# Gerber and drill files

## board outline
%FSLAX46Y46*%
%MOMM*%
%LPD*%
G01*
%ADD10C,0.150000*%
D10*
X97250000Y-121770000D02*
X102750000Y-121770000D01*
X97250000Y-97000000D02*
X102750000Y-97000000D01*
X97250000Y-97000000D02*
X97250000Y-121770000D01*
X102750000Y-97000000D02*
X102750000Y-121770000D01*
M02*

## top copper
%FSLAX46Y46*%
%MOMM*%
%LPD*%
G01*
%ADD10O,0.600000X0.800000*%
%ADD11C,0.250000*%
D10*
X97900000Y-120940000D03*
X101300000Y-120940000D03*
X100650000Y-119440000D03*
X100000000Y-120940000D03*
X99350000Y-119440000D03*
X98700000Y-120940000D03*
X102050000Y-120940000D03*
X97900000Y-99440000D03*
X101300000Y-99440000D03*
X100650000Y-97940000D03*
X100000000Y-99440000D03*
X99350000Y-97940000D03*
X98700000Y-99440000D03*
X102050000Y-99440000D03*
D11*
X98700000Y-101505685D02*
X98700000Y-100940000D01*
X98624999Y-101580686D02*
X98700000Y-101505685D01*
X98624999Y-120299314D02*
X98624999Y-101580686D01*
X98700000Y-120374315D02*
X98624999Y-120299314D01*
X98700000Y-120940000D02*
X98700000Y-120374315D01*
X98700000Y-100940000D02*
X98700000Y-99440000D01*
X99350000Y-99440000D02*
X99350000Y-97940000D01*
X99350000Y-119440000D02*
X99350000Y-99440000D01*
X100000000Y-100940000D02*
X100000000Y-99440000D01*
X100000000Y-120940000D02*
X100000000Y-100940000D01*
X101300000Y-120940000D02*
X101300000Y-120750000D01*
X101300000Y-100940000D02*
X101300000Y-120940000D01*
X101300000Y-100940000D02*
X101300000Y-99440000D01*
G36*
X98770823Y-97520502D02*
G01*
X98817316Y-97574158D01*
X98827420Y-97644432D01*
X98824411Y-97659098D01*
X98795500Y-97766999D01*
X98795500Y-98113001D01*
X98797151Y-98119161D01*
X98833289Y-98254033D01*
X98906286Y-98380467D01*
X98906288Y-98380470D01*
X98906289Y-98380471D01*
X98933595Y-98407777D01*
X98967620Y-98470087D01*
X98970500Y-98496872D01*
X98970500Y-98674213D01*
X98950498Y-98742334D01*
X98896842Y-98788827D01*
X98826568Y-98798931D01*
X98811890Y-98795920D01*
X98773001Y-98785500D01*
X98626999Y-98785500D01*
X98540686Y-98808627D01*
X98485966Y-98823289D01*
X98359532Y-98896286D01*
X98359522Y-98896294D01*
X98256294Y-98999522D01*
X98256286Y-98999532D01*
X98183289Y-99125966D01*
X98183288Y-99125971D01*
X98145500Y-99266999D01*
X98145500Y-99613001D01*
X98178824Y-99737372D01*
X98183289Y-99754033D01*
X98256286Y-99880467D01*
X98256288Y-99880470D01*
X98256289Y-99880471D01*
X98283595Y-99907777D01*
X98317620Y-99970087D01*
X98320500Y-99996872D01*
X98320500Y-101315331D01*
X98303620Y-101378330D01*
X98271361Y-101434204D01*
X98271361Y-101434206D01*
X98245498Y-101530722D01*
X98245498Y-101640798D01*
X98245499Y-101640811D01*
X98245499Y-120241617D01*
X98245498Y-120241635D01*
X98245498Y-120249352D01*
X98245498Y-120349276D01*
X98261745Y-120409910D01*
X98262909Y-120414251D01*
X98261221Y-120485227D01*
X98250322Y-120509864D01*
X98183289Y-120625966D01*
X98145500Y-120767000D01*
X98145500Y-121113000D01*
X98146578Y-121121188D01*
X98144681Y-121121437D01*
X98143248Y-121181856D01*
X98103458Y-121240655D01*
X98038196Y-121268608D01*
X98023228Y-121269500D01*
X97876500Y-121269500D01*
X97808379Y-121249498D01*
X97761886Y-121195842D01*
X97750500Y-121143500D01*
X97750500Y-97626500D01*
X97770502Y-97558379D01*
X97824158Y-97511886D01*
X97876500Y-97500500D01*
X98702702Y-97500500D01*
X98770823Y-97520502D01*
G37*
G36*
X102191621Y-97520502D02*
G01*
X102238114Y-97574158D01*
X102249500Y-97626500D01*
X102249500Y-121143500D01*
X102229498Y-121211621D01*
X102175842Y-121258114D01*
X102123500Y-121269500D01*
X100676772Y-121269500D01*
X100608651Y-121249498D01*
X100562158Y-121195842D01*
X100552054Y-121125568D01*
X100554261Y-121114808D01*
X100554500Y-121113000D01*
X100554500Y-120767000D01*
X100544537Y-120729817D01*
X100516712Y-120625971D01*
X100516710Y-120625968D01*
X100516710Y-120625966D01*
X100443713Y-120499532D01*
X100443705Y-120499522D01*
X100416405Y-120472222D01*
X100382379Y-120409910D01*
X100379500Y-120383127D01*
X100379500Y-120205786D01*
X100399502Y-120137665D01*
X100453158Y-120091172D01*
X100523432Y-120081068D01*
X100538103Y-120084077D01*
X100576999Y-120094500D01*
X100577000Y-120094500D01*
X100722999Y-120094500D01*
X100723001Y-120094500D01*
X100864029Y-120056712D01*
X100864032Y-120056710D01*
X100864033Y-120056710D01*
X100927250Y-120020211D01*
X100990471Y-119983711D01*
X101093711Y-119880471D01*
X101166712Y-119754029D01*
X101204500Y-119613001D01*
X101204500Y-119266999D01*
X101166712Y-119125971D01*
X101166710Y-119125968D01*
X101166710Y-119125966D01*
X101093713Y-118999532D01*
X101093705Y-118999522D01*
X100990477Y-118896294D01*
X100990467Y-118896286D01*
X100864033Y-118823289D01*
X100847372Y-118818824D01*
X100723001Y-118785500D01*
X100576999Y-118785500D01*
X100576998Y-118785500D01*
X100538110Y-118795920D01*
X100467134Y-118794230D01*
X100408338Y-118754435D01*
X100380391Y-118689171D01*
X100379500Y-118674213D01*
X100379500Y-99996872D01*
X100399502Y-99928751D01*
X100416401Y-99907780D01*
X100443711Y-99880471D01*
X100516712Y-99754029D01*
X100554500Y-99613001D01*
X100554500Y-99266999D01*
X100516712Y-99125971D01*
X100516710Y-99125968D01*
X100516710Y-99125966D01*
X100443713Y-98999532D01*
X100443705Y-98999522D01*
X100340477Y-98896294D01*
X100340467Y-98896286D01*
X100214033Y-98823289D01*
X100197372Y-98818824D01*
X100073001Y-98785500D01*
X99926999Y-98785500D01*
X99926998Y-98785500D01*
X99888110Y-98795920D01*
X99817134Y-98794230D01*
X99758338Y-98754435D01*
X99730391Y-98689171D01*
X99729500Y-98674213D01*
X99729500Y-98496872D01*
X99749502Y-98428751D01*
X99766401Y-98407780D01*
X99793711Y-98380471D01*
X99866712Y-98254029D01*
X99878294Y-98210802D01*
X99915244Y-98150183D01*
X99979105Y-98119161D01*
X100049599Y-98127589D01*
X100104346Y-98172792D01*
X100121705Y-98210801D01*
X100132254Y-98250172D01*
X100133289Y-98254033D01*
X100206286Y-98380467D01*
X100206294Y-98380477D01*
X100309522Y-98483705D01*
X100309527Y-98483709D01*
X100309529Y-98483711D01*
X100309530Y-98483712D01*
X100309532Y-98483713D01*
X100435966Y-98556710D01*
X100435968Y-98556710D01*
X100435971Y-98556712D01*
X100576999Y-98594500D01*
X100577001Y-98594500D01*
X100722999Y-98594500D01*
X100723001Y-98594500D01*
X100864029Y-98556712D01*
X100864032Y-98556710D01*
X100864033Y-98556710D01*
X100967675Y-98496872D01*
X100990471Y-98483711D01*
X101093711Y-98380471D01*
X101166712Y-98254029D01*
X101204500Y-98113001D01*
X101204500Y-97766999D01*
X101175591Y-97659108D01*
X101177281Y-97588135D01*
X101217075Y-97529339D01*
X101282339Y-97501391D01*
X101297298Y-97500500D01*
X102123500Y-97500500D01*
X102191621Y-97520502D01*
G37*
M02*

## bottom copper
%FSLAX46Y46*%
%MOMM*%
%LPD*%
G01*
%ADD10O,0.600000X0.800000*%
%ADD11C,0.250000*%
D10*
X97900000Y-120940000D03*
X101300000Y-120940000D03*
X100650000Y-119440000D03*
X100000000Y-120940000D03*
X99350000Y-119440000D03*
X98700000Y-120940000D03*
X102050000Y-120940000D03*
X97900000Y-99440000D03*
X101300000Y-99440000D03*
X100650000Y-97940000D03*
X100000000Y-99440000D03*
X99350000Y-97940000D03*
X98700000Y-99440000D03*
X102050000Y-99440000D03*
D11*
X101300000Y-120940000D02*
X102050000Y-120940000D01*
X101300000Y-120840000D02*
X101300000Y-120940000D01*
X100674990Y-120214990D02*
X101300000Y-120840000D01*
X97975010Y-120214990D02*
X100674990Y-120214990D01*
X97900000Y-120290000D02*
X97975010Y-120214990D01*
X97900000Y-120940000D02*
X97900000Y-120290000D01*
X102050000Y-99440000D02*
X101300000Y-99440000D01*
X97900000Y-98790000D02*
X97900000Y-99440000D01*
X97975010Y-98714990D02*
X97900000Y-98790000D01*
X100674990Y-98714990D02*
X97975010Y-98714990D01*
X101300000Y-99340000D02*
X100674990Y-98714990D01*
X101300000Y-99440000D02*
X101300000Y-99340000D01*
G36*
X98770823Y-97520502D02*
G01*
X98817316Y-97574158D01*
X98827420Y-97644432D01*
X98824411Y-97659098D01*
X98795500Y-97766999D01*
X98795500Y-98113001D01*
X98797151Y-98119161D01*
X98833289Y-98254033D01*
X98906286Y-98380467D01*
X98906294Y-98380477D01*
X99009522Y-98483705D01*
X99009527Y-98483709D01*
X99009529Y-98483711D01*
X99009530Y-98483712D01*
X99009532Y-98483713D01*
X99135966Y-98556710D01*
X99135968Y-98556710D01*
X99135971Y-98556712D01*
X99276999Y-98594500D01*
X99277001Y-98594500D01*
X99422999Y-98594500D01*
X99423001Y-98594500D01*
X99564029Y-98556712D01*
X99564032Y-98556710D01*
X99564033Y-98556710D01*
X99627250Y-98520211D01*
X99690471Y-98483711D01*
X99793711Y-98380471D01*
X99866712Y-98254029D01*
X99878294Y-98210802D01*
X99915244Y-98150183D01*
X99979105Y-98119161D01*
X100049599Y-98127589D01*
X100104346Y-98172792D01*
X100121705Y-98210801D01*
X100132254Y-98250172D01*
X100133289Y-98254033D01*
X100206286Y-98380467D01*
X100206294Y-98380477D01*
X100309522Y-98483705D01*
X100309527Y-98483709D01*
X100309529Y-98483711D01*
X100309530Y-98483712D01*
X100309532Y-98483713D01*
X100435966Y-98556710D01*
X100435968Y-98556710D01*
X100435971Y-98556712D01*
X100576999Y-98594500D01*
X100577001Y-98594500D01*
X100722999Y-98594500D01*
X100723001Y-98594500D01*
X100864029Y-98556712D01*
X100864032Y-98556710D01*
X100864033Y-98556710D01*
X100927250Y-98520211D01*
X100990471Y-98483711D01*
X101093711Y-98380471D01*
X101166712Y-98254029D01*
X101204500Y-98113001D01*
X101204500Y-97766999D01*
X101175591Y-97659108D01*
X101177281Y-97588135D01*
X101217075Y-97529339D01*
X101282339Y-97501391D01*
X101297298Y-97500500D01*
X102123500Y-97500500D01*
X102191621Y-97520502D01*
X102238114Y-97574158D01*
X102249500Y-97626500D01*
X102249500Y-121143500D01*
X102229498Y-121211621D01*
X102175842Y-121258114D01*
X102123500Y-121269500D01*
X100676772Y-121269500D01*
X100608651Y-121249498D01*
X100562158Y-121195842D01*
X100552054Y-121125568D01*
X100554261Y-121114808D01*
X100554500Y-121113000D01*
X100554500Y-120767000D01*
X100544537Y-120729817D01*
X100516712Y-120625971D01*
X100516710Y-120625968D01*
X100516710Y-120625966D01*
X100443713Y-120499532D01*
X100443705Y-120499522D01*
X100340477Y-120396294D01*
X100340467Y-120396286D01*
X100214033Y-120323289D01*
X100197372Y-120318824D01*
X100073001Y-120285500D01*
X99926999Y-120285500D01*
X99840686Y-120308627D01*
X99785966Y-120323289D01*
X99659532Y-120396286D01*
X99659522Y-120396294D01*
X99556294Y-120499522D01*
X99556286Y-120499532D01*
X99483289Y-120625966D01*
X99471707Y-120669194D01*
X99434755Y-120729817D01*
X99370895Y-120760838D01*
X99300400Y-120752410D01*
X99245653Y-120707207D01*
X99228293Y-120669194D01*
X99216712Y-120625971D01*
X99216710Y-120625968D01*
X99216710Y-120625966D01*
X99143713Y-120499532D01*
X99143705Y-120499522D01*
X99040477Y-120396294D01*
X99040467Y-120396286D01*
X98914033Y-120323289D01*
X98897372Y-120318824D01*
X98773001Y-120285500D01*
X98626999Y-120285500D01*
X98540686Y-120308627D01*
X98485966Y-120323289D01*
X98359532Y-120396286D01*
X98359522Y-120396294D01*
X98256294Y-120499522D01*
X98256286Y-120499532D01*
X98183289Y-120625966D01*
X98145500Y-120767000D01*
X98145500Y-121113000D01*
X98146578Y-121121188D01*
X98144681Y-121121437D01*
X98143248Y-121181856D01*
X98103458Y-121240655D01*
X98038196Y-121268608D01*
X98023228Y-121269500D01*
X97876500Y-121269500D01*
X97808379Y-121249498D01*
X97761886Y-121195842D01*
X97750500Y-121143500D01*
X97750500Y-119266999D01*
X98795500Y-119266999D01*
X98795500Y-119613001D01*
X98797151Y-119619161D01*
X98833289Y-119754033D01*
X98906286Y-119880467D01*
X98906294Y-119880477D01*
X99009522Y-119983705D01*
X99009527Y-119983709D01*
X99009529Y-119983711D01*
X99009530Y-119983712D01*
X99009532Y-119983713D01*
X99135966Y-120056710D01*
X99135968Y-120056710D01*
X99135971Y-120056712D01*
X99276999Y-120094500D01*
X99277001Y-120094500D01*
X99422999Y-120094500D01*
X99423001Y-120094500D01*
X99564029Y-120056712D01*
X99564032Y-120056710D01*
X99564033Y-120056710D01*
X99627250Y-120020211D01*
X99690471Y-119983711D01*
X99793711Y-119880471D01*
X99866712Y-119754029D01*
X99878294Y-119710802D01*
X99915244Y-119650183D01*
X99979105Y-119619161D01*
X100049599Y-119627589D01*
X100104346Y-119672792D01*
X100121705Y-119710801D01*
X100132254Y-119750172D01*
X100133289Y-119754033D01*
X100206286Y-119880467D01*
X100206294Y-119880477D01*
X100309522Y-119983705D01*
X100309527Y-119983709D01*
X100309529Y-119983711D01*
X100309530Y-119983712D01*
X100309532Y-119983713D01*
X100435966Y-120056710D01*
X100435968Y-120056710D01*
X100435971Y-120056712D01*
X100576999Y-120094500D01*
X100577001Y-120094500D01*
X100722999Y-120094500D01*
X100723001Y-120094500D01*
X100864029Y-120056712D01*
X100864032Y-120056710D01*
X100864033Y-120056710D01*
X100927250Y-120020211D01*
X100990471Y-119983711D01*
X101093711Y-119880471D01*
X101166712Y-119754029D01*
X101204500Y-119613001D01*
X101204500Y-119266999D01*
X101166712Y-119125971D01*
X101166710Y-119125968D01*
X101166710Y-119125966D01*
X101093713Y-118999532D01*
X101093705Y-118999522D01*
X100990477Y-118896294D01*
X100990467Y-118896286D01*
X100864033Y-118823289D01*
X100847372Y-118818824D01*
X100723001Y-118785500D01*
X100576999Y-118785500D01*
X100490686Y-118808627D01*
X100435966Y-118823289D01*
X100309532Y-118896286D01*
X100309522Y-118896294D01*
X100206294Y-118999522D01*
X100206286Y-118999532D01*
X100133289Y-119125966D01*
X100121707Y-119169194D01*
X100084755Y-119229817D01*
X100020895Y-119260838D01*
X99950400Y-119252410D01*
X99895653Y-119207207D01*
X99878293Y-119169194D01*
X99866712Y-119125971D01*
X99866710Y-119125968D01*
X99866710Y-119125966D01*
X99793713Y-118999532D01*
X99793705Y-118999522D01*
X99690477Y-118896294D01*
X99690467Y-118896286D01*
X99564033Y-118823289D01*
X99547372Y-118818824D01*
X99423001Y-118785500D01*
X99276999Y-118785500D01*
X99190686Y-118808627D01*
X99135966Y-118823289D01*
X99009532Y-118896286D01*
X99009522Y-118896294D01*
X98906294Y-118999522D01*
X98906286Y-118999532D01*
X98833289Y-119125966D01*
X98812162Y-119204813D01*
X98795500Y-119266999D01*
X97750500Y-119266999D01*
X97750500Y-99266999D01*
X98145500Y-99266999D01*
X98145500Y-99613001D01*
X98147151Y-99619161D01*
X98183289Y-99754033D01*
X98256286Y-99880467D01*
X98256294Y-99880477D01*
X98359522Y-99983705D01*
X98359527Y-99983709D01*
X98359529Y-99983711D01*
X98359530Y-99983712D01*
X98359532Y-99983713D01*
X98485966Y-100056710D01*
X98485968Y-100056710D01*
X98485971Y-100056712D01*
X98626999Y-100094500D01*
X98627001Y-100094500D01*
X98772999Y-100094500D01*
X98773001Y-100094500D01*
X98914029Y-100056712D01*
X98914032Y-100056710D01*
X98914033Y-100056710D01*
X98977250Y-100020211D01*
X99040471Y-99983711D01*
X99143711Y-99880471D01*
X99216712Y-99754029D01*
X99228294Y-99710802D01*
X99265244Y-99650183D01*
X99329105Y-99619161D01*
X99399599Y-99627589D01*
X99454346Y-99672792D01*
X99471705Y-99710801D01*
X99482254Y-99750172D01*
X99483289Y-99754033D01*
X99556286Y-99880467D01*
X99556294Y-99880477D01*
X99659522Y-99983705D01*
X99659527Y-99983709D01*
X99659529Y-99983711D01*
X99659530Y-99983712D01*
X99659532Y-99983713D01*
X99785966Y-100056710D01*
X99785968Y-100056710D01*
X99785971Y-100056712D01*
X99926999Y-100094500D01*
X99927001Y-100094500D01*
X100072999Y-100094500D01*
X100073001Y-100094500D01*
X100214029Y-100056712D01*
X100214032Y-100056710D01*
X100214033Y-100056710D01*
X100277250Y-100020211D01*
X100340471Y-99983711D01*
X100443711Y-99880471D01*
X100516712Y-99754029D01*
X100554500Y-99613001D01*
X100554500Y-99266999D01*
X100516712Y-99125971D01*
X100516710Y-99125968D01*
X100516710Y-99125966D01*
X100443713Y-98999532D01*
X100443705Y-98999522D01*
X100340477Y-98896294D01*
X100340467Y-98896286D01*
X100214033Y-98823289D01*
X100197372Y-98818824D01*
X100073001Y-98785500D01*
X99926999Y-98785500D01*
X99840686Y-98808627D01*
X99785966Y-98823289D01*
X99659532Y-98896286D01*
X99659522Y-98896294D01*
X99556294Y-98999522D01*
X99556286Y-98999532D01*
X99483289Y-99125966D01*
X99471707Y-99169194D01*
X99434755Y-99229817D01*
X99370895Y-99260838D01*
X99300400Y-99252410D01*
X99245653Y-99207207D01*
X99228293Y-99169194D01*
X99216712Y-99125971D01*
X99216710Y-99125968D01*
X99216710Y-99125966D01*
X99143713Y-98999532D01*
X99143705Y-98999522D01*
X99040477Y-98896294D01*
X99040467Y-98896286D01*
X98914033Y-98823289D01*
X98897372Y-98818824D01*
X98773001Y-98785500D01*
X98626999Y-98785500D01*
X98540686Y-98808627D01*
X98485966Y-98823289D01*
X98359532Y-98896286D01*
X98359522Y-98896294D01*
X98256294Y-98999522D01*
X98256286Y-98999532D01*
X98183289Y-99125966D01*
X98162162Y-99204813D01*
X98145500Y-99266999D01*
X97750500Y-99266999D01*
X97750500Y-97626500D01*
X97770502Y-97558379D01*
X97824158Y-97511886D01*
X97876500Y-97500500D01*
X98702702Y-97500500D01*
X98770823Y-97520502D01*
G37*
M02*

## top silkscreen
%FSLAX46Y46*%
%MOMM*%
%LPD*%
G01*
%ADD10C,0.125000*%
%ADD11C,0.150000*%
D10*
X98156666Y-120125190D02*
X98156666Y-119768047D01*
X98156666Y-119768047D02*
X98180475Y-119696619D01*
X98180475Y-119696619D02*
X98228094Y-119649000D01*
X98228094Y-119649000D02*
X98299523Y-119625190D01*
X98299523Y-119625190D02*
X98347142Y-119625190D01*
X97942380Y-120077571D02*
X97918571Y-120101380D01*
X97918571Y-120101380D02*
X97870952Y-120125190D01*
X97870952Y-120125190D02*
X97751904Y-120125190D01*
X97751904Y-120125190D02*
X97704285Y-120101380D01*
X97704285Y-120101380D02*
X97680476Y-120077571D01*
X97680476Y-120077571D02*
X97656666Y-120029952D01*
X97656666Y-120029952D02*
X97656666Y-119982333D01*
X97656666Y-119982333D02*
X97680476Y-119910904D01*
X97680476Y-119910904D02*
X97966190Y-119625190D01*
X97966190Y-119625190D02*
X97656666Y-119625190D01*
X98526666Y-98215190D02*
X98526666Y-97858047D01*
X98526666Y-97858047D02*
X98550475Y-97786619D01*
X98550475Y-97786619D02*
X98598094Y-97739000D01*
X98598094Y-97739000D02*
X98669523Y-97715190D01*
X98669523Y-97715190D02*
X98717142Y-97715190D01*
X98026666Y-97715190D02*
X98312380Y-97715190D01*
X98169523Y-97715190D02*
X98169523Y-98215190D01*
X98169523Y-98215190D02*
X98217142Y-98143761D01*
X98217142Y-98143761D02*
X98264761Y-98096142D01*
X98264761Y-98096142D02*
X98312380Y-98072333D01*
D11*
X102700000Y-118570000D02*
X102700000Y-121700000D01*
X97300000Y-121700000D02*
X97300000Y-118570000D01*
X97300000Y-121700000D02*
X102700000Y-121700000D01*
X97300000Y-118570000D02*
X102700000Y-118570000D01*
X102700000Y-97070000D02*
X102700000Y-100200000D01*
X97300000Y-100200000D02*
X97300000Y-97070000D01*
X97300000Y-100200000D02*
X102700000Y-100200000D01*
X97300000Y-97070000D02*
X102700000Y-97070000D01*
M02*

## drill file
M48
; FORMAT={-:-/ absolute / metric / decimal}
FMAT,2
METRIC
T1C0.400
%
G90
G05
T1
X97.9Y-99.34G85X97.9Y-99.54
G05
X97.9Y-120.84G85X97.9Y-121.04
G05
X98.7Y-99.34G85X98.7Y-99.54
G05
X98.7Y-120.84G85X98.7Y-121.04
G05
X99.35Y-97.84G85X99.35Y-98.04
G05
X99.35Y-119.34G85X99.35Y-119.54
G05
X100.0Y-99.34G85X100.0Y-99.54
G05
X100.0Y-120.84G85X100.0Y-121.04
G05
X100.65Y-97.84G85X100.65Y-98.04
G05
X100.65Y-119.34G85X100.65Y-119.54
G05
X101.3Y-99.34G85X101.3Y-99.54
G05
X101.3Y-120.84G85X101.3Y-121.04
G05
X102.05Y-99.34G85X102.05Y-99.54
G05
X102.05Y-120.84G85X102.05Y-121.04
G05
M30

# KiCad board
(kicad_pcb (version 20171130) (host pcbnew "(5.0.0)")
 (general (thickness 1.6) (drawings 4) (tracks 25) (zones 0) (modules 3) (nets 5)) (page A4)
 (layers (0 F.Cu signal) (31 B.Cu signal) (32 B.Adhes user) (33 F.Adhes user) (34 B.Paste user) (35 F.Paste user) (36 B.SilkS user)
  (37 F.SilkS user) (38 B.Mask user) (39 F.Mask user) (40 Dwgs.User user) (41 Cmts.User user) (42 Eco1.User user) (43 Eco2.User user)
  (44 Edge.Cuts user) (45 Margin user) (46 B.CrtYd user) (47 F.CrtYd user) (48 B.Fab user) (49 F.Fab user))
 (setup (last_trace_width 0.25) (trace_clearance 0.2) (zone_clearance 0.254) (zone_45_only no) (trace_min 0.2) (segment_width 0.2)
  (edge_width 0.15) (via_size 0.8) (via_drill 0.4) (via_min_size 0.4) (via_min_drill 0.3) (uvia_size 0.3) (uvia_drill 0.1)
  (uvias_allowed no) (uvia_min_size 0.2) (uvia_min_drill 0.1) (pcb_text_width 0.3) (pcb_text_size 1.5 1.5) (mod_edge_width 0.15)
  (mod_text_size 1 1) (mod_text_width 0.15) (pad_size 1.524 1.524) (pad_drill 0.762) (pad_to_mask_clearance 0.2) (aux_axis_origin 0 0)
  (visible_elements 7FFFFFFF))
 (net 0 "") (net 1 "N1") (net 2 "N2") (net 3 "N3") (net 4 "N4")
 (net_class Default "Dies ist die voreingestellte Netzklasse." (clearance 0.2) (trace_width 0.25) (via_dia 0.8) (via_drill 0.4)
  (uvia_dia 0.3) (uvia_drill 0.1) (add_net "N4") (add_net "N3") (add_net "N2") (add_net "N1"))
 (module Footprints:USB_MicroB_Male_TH (layer F.Cu) (at 100 120)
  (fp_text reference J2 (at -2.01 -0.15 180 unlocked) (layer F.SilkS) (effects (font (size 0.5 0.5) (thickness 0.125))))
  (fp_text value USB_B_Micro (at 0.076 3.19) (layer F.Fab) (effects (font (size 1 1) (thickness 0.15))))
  (fp_line (start 2.7 -1.43) (end 2.7 1.7) (layer F.SilkS) (width 0.15))
  (fp_line (start -2.7 1.7) (end -2.7 -1.43) (layer F.SilkS) (width 0.15))
  (fp_line (start -2.7 1.7) (end 2.7 1.7) (layer F.SilkS) (width 0.15))
  (fp_line (start -2.7 -1.43) (end 2.7 -1.43) (layer F.SilkS) (width 0.15))
  (pad 6 thru_hole oval (at -2.1 0.94) (size 0.6 0.8) (drill oval 0.4 0.6) (layers *.Cu *.Mask) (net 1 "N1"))
  (pad 5 thru_hole oval (at 1.3 0.94) (size 0.6 0.8) (drill oval 0.4 0.6) (layers *.Cu *.Mask) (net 1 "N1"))
  (pad 4 thru_hole oval (at 0.65 -0.56) (size 0.6 0.8) (drill oval 0.4 0.6) (layers *.Cu *.Mask))
  (pad 3 thru_hole oval (at 0 0.94) (size 0.6 0.8) (drill oval 0.4 0.6) (layers *.Cu *.Mask) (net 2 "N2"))
  (pad 2 thru_hole oval (at -0.65 -0.56) (size 0.6 0.8) (drill oval 0.4 0.6) (layers *.Cu *.Mask) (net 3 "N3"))
  (pad 1 thru_hole oval (at -1.3 0.94) (size 0.6 0.8) (drill oval 0.4 0.6) (layers *.Cu *.Mask) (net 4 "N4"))
  (pad 6 thru_hole oval (at 2.05 0.94) (size 0.6 0.8) (drill oval 0.4 0.6) (layers *.Cu *.Mask) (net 1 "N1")))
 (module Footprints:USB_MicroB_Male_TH (layer F.Cu) (at 100 98.5)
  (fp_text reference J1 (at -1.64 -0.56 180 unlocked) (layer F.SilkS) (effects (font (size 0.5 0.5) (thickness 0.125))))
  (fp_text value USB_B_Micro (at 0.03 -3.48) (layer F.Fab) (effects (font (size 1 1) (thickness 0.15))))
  (fp_line (start 2.7 -1.43) (end 2.7 1.7) (layer F.SilkS) (width 0.15))
  (fp_line (start -2.7 1.7) (end -2.7 -1.43) (layer F.SilkS) (width 0.15))
  (fp_line (start -2.7 1.7) (end 2.7 1.7) (layer F.SilkS) (width 0.15))
  (fp_line (start -2.7 -1.43) (end 2.7 -1.43) (layer F.SilkS) (width 0.15))
  (pad 6 thru_hole oval (at -2.1 0.94) (size 0.6 0.8) (drill oval 0.4 0.6) (layers *.Cu *.Mask) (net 1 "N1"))
  (pad 5 thru_hole oval (at 1.3 0.94) (size 0.6 0.8) (drill oval 0.4 0.6) (layers *.Cu *.Mask) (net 1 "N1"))
  (pad 4 thru_hole oval (at 0.65 -0.56) (size 0.6 0.8) (drill oval 0.4 0.6) (layers *.Cu *.Mask))
  (pad 3 thru_hole oval (at 0 0.94) (size 0.6 0.8) (drill oval 0.4 0.6) (layers *.Cu *.Mask) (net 2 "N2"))
  (pad 2 thru_hole oval (at -0.65 -0.56) (size 0.6 0.8) (drill oval 0.4 0.6) (layers *.Cu *.Mask) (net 3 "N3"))
  (pad 1 thru_hole oval (at -1.3 0.94) (size 0.6 0.8) (drill oval 0.4 0.6) (layers *.Cu *.Mask) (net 4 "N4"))
  (pad 6 thru_hole oval (at 2.05 0.94) (size 0.6 0.8) (drill oval 0.4 0.6) (layers *.Cu *.Mask) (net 1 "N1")))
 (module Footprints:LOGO (layer B.Cu) (at 100.36 109.2 90)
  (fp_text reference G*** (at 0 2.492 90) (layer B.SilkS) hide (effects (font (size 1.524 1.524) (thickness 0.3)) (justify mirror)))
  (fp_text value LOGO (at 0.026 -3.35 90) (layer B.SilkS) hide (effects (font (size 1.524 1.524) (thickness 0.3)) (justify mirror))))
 (gr_line (start 97.25 121.77) (end 102.75 121.77) (layer Edge.Cuts) (width 0.15))
 (gr_line (start 97.25 97) (end 102.75 97) (layer Edge.Cuts) (width 0.15))
 (gr_line (start 97.25 97) (end 97.25 121.77) (layer Edge.Cuts) (width 0.15))
 (gr_line (start 102.75 97) (end 102.75 121.77) (layer Edge.Cuts) (width 0.15))
 (segment (start 98.7 101.505685) (end 98.7 100.94) (width 0.25) (layer F.Cu) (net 4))
 (segment (start 98.624999 101.580686) (end 98.7 101.505685) (width 0.25) (layer F.Cu) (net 4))
 (segment (start 98.624999 120.299314) (end 98.624999 101.580686) (width 0.25) (layer F.Cu) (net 4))
 (segment (start 98.7 120.374315) (end 98.624999 120.299314) (width 0.25) (layer F.Cu) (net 4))
 (segment (start 98.7 120.94) (end 98.7 120.374315) (width 0.25) (layer F.Cu) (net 4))
 (segment (start 98.7 100.94) (end 98.7 99.44) (width 0.25) (layer F.Cu) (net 4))
 (segment (start 99.35 99.44) (end 99.35 97.94) (width 0.25) (layer F.Cu) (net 3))
 (segment (start 99.35 119.44) (end 99.35 99.44) (width 0.25) (layer F.Cu) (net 3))
 (segment (start 100 100.94) (end 100 99.44) (width 0.25) (layer F.Cu) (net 2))
 (segment (start 100 120.94) (end 100 100.94) (width 0.25) (layer F.Cu) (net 2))
 (segment (start 101.3 120.94) (end 101.3 120.75) (width 0.25) (layer F.Cu) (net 1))
 (segment (start 101.3 120.94) (end 102.05 120.94) (width 0.25) (layer B.Cu) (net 1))
 (segment (start 101.3 100.94) (end 101.3 120.94) (width 0.25) (layer F.Cu) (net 1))
 (segment (start 101.3 120.84) (end 101.3 120.94) (width 0.25) (layer B.Cu) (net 1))
 (segment (start 100.67499 120.21499) (end 101.3 120.84) (width 0.25) (layer B.Cu) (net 1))
 (segment (start 97.97501 120.21499) (end 100.67499 120.21499) (width 0.25) (layer B.Cu) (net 1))
 (segment (start 97.9 120.29) (end 97.97501 120.21499) (width 0.25) (layer B.Cu) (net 1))
 (segment (start 97.9 120.94) (end 97.9 120.29) (width 0.25) (layer B.Cu) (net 1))
 (segment (start 101.3 100.94) (end 101.3 99.44) (width 0.25) (layer F.Cu) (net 1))
 (segment (start 102.05 99.44) (end 101.3 99.44) (width 0.25) (layer B.Cu) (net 1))
 (segment (start 97.9 98.79) (end 97.9 99.44) (width 0.25) (layer B.Cu) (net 1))
 (segment (start 97.97501 98.71499) (end 97.9 98.79) (width 0.25) (layer B.Cu) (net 1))
 (segment (start 100.67499 98.71499) (end 97.97501 98.71499) (width 0.25) (layer B.Cu) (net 1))
 (segment (start 101.3 99.34) (end 100.67499 98.71499) (width 0.25) (layer B.Cu) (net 1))
 (segment (start 101.3 99.44) (end 101.3 99.34) (width 0.25) (layer B.Cu) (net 1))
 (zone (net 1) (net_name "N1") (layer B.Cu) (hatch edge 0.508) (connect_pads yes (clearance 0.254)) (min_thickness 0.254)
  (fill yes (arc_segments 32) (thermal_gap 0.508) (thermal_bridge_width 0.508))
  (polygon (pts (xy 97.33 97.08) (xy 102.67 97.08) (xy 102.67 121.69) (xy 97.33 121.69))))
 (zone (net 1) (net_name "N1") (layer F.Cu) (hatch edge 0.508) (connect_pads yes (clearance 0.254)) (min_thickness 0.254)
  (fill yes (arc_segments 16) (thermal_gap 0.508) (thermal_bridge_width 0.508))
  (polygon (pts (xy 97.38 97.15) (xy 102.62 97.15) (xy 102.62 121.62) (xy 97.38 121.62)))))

